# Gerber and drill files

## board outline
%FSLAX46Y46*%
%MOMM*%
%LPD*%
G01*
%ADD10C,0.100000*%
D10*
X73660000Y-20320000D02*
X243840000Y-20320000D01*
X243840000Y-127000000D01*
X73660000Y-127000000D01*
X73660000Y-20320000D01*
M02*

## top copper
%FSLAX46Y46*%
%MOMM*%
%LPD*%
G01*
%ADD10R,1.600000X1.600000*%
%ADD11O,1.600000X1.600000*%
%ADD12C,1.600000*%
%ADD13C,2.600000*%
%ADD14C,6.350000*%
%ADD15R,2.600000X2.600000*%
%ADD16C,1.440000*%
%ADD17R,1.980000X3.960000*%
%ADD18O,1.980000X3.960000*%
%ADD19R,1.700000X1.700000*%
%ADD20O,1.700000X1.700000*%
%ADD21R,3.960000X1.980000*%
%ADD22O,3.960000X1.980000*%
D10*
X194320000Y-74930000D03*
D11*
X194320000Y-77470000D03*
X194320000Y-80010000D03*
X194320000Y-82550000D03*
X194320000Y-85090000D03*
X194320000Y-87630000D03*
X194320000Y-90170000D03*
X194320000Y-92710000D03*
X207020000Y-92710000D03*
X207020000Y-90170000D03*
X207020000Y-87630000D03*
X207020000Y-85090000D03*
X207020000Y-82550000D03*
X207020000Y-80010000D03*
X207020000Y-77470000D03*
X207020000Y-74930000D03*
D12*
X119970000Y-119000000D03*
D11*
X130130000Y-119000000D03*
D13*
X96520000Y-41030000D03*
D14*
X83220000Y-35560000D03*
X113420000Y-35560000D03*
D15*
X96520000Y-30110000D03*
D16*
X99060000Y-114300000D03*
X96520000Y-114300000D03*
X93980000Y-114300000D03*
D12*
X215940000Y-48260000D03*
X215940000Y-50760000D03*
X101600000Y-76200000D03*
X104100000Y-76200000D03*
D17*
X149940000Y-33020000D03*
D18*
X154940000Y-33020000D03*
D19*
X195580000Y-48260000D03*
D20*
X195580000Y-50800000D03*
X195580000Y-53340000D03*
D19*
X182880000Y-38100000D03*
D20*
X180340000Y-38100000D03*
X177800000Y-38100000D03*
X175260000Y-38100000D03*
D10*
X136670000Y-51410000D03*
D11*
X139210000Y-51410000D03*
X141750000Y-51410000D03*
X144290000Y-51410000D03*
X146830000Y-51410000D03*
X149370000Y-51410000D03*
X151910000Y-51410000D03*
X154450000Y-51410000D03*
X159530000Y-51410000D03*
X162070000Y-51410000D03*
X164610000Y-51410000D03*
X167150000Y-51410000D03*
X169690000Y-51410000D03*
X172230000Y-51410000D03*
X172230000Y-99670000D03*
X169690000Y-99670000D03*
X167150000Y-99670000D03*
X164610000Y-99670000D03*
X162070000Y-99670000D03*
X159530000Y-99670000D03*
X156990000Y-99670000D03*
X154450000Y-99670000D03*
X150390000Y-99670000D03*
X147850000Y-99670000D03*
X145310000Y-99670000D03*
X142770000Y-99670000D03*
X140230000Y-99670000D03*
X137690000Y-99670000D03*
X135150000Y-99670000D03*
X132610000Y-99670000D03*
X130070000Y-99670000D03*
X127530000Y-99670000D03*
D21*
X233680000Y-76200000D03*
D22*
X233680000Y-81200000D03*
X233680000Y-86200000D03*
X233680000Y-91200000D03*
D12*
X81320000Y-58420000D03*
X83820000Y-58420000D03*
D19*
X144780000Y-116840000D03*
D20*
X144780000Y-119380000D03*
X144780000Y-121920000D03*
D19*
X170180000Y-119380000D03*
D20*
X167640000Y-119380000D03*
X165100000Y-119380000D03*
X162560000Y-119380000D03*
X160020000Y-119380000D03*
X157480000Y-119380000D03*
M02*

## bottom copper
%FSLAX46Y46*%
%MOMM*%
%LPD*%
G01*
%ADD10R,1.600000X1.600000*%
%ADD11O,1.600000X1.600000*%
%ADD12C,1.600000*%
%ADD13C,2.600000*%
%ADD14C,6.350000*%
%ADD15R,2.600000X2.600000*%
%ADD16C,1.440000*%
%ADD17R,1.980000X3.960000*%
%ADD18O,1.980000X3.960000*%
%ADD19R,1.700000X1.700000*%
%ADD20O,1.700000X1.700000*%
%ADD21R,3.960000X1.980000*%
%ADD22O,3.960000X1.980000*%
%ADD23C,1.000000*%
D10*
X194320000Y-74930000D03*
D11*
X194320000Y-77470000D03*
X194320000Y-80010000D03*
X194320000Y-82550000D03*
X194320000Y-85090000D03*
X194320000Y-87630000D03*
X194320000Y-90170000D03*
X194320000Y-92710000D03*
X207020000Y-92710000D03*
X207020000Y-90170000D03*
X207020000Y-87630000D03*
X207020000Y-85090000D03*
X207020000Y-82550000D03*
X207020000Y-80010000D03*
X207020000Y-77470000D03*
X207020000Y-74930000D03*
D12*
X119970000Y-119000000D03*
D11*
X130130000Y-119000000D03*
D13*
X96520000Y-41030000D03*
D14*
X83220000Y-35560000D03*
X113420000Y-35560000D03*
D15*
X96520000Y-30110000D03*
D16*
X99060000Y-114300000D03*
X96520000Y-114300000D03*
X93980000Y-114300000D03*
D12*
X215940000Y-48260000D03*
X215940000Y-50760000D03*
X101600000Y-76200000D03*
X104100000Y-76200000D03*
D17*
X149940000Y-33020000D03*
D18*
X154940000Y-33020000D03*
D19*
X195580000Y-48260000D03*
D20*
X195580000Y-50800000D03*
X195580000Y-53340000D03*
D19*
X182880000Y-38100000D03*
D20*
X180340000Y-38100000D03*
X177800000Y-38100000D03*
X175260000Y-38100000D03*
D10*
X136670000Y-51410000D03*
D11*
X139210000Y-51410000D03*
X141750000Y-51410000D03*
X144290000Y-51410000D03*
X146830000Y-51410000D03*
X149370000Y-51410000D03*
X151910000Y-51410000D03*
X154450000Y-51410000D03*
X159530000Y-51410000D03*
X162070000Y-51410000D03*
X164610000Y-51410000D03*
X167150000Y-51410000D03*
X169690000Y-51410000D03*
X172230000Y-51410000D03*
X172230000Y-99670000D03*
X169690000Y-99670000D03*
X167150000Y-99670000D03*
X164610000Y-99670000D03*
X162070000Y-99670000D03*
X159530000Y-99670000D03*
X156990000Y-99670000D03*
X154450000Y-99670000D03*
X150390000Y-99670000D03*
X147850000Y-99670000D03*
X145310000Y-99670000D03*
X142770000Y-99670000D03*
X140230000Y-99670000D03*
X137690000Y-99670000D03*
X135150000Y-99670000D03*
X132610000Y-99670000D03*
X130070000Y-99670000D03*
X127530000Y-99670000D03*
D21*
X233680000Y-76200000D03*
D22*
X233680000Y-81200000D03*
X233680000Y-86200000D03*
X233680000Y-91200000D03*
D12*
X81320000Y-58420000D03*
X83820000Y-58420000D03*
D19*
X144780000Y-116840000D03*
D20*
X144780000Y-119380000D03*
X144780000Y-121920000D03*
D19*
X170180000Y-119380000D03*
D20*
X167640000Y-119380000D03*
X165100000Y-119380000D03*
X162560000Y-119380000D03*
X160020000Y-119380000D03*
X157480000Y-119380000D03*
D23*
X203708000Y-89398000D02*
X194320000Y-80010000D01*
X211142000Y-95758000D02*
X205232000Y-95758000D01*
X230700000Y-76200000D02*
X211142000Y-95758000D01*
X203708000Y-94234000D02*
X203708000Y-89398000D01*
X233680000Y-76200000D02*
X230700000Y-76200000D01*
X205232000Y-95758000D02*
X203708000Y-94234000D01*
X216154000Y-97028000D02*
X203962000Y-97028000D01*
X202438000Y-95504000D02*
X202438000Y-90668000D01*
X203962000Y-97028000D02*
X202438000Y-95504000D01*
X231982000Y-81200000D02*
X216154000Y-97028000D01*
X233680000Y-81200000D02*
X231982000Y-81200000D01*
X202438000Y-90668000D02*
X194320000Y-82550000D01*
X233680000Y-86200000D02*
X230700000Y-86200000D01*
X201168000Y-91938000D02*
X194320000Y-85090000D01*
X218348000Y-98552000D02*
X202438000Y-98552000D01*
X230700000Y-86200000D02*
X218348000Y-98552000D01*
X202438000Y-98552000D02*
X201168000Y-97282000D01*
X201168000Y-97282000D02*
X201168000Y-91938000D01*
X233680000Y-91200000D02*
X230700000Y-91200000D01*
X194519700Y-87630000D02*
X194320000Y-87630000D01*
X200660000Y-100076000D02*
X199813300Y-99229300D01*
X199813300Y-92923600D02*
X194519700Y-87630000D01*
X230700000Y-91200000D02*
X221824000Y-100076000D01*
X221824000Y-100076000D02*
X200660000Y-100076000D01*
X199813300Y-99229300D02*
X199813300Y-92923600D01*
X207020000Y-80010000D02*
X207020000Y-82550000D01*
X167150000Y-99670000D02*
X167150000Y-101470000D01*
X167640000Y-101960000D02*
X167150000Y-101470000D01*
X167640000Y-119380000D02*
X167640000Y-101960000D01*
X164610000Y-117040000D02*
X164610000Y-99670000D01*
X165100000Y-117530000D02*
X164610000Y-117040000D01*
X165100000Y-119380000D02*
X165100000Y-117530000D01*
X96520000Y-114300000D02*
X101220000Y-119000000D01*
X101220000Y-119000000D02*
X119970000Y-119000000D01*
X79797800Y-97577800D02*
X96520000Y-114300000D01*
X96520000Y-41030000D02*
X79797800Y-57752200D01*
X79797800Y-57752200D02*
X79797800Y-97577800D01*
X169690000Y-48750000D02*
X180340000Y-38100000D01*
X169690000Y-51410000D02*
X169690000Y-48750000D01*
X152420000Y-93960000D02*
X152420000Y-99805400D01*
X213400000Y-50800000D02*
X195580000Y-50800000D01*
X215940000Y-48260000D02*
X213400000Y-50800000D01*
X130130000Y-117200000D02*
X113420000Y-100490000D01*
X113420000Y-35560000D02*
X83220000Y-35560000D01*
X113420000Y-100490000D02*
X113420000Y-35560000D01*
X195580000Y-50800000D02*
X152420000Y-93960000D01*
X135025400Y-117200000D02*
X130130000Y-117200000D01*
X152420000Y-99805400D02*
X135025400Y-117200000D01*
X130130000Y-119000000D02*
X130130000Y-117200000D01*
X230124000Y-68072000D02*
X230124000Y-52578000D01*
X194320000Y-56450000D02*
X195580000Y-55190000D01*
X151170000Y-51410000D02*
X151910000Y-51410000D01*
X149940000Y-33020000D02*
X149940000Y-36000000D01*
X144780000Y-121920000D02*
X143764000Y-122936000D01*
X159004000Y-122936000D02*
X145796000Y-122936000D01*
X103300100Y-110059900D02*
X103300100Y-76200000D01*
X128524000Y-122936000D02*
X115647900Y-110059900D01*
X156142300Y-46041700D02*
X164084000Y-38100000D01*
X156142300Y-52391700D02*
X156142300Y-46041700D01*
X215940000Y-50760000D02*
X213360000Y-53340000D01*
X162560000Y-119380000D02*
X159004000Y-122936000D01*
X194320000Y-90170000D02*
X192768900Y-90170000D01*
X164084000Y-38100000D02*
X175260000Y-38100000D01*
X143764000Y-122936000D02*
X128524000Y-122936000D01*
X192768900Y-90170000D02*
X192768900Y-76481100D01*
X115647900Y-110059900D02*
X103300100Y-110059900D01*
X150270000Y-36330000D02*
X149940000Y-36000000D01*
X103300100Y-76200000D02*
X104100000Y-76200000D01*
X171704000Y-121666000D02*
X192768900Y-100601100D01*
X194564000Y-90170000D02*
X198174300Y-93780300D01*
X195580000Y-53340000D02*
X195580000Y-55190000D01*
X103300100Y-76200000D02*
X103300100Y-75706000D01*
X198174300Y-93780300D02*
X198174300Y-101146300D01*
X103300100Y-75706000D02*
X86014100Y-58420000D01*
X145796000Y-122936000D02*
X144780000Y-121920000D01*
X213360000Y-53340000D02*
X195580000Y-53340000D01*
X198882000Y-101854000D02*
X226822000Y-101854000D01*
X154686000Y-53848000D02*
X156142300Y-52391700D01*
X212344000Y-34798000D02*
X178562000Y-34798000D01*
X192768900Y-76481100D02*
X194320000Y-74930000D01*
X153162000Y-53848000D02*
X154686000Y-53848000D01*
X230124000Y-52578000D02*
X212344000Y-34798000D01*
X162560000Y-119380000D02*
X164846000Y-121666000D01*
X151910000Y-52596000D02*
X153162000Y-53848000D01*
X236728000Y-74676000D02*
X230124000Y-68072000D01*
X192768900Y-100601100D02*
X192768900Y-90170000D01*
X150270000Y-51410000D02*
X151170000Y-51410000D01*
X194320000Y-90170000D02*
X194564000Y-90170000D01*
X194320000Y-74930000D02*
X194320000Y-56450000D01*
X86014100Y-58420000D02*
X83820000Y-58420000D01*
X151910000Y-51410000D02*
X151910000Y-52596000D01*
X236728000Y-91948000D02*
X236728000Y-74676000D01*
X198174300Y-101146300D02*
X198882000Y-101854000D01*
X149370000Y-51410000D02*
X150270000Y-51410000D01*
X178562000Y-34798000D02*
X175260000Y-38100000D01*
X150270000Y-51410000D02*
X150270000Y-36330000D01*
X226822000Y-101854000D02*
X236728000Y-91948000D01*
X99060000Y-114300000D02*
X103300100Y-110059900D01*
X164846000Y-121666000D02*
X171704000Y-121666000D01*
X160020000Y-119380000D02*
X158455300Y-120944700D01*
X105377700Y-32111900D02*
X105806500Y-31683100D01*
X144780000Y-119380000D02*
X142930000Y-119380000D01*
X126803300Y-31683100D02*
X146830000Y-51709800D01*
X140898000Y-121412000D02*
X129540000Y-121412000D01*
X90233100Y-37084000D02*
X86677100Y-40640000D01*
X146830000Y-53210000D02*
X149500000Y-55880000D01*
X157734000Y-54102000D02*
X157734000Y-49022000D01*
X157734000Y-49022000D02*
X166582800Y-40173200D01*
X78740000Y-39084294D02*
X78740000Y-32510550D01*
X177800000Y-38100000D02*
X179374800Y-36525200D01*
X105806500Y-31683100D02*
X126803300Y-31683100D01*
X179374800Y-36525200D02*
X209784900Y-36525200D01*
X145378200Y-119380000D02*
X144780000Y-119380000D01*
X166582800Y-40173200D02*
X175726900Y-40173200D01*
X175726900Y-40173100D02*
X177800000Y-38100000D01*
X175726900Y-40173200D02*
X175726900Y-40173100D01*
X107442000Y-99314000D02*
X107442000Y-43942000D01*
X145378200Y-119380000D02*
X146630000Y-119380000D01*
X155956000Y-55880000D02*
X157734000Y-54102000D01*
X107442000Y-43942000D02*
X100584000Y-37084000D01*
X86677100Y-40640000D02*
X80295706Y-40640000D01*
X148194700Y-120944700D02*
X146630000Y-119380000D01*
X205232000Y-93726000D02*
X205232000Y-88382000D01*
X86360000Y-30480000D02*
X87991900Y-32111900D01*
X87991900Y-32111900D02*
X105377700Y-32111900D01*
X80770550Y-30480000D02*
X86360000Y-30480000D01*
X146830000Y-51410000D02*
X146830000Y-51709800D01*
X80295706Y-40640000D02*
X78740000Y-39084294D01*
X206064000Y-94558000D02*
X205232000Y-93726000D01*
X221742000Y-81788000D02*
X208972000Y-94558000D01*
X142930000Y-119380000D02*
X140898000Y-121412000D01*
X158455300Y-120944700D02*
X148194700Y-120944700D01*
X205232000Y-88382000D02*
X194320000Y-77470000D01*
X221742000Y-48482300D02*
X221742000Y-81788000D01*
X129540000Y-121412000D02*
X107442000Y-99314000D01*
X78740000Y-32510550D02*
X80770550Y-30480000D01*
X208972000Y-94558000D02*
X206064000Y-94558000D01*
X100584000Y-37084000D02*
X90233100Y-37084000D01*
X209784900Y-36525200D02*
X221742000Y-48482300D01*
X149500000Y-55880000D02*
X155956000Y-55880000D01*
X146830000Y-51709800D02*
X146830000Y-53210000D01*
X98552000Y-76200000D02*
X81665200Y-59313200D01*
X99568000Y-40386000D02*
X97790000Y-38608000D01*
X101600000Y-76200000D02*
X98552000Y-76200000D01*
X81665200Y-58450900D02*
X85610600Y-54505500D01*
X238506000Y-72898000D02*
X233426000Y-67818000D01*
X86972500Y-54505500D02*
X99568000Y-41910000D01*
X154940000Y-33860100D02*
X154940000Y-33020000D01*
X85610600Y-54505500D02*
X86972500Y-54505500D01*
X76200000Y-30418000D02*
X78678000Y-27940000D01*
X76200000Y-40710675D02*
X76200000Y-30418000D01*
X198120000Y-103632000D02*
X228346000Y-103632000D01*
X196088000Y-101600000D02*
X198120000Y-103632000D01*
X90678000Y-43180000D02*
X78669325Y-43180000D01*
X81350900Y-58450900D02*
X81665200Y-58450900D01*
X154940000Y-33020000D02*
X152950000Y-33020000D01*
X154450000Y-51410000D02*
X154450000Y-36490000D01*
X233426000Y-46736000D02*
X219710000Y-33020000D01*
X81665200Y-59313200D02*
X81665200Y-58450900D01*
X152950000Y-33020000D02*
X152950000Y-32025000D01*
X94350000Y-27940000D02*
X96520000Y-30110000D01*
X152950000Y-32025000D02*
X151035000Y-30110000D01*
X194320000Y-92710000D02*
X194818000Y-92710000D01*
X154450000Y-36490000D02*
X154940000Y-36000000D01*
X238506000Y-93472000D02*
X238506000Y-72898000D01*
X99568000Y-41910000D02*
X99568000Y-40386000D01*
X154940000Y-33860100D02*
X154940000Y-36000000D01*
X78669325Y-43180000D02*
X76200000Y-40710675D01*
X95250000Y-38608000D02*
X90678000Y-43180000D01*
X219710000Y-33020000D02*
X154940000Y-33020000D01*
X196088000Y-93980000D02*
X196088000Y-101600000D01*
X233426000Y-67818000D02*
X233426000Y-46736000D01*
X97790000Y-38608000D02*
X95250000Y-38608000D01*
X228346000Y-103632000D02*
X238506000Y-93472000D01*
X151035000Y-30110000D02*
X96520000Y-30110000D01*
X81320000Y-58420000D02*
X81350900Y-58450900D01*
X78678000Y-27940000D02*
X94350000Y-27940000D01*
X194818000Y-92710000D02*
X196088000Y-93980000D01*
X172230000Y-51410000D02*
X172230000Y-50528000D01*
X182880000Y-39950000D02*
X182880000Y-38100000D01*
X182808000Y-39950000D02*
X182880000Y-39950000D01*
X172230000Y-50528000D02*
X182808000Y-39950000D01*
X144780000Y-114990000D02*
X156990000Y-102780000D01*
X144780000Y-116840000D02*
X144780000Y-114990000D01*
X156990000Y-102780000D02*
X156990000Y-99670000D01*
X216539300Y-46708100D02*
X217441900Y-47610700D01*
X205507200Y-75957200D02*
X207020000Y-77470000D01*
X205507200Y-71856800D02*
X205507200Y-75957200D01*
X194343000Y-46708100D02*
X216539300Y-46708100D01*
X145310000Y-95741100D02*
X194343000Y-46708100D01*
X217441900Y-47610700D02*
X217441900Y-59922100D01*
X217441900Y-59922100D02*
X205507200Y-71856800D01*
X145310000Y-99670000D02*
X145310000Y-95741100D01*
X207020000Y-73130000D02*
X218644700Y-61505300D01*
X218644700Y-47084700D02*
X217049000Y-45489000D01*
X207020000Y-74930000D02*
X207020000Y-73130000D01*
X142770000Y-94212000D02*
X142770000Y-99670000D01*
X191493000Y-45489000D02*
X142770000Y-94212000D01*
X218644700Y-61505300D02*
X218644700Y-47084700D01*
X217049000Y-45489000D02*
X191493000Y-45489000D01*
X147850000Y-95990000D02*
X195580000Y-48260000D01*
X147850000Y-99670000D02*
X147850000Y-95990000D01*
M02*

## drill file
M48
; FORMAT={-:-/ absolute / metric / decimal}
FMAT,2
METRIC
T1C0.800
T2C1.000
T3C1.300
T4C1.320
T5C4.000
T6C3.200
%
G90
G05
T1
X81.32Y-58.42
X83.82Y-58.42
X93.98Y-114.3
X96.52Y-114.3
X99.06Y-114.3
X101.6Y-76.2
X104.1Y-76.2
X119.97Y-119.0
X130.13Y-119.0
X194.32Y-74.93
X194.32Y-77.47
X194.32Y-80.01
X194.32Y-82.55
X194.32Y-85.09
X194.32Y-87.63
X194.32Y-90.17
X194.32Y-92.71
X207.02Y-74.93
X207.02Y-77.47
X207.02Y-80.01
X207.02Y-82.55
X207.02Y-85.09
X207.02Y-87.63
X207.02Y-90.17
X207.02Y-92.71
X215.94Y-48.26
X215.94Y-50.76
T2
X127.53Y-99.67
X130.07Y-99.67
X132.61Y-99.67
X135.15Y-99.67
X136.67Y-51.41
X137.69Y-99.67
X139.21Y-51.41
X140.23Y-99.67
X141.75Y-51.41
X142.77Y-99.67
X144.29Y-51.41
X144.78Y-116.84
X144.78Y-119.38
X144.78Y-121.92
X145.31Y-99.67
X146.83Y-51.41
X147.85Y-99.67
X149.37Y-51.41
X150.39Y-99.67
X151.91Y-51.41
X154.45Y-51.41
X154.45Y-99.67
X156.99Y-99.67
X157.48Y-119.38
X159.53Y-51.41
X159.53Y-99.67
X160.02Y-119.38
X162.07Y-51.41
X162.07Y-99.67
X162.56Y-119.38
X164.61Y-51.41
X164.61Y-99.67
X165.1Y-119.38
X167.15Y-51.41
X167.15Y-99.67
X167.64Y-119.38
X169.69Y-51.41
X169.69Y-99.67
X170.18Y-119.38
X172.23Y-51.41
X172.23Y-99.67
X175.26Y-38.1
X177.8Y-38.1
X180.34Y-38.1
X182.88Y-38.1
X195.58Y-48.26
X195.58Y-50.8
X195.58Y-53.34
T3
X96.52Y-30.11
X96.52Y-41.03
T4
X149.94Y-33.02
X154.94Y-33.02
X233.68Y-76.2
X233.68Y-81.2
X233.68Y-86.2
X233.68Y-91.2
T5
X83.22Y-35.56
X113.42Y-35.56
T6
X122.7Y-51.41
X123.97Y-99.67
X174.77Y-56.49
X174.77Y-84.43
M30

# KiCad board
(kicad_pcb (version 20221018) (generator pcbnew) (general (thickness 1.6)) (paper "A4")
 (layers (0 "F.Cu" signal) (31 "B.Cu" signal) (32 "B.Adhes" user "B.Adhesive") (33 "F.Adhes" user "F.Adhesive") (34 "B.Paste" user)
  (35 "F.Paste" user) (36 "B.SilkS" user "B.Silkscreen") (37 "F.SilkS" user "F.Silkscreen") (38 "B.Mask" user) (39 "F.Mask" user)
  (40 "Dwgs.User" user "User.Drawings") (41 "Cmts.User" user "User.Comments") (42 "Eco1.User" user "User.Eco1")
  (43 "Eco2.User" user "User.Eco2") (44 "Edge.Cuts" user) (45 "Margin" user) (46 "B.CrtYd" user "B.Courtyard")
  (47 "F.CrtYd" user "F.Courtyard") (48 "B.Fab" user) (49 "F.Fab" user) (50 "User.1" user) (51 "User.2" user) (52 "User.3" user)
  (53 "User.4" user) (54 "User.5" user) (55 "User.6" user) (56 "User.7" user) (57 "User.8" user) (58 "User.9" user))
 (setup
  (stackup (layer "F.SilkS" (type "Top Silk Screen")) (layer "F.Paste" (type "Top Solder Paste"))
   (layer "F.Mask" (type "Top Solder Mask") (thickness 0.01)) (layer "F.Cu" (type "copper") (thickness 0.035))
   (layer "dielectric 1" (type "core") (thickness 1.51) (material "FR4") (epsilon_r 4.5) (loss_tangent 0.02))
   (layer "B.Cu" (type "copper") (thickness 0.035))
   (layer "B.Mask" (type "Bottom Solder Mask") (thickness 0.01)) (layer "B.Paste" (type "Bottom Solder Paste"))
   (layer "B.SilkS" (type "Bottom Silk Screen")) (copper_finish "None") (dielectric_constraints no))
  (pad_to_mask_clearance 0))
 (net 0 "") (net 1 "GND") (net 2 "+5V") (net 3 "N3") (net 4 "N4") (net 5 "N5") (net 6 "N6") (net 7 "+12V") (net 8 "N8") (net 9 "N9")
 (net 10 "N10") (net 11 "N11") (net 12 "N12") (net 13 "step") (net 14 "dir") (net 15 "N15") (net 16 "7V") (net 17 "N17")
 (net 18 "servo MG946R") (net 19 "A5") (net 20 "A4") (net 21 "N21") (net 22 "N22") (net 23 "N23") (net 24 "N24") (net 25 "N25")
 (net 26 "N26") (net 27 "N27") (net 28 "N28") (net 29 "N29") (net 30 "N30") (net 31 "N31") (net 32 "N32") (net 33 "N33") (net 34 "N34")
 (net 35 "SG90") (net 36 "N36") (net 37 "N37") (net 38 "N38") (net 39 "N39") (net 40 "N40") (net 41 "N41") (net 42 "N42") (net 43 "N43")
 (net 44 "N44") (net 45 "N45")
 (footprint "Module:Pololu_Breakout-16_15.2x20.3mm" (layer "F.Cu") (at 194.32 74.93)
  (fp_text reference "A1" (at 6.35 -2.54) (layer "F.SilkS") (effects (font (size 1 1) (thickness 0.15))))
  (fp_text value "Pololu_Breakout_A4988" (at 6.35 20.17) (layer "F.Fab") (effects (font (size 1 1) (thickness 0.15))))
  (pad "1" thru_hole rect (at 0 0) (size 1.6 1.6) (drill 0.8) (layers "*.Cu" "*.Mask") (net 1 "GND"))
  (pad "2" thru_hole oval (at 0 2.54) (size 1.6 1.6) (drill 0.8) (layers "*.Cu" "*.Mask") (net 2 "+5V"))
  (pad "3" thru_hole oval (at 0 5.08) (size 1.6 1.6) (drill 0.8) (layers "*.Cu" "*.Mask") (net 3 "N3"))
  (pad "4" thru_hole oval (at 0 7.62) (size 1.6 1.6) (drill 0.8) (layers "*.Cu" "*.Mask") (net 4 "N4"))
  (pad "5" thru_hole oval (at 0 10.16) (size 1.6 1.6) (drill 0.8) (layers "*.Cu" "*.Mask") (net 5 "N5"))
  (pad "6" thru_hole oval (at 0 12.7) (size 1.6 1.6) (drill 0.8) (layers "*.Cu" "*.Mask") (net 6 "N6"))
  (pad "7" thru_hole oval (at 0 15.24) (size 1.6 1.6) (drill 0.8) (layers "*.Cu" "*.Mask") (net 1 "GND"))
  (pad "8" thru_hole oval (at 0 17.78) (size 1.6 1.6) (drill 0.8) (layers "*.Cu" "*.Mask") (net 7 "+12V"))
  (pad "9" thru_hole oval (at 12.7 17.78) (size 1.6 1.6) (drill 0.8) (layers "*.Cu" "*.Mask") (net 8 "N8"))
  (pad "10" thru_hole oval (at 12.7 15.24) (size 1.6 1.6) (drill 0.8) (layers "*.Cu" "*.Mask") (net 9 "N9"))
  (pad "11" thru_hole oval (at 12.7 12.7) (size 1.6 1.6) (drill 0.8) (layers "*.Cu" "*.Mask") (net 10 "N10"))
  (pad "12" thru_hole oval (at 12.7 10.16) (size 1.6 1.6) (drill 0.8) (layers "*.Cu" "*.Mask") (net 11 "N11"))
  (pad "13" thru_hole oval (at 12.7 7.62) (size 1.6 1.6) (drill 0.8) (layers "*.Cu" "*.Mask") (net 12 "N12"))
  (pad "14" thru_hole oval (at 12.7 5.08) (size 1.6 1.6) (drill 0.8) (layers "*.Cu" "*.Mask") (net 12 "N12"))
  (pad "15" thru_hole oval (at 12.7 2.54) (size 1.6 1.6) (drill 0.8) (layers "*.Cu" "*.Mask") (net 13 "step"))
  (pad "16" thru_hole oval (at 12.7 0) (size 1.6 1.6) (drill 0.8) (layers "*.Cu" "*.Mask") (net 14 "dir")))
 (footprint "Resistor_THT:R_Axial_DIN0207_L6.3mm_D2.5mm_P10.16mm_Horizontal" (layer "F.Cu") (at 119.97 119)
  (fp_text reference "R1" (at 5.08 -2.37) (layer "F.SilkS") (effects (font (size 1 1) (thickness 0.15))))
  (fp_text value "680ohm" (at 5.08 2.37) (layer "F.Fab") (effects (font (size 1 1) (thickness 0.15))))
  (pad "1" thru_hole circle (at 0 0) (size 1.6 1.6) (drill 0.8) (layers "*.Cu" "*.Mask") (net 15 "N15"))
  (pad "2" thru_hole oval (at 10.16 0) (size 1.6 1.6) (drill 0.8) (layers "*.Cu" "*.Mask") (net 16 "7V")))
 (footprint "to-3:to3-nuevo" (layer "F.Cu") (at 98.74 32.39)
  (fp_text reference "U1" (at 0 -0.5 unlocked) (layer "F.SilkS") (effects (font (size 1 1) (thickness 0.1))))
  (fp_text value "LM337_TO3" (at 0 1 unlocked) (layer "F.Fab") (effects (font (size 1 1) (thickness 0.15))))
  (pad "1" thru_hole circle (at -2.22 8.64) (size 2.6 2.6) (drill 1.3) (layers "*.Cu" "*.Mask") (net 15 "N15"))
  (pad "2" thru_hole circle (at -15.52 3.17) (size 6.35 6.35) (drill 4) (layers "*.Cu" "*.Mask") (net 16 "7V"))
  (pad "2" thru_hole circle (at 14.68 3.17) (size 6.35 6.35) (drill 4) (layers "*.Cu" "*.Mask") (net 16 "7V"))
  (pad "3" thru_hole rect (at -2.22 -2.28) (size 2.6 2.6) (drill 1.3) (layers "*.Cu" "*.Mask") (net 7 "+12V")))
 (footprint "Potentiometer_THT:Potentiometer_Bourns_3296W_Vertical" (layer "F.Cu") (at 99.06 114.3)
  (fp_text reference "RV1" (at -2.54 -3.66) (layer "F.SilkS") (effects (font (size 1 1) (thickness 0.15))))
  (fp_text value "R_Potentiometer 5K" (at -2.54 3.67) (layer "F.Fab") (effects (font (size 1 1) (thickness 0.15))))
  (pad "1" thru_hole circle (at 0 0) (size 1.44 1.44) (drill 0.8) (layers "*.Cu" "*.Mask") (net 1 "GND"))
  (pad "2" thru_hole circle (at -2.54 0) (size 1.44 1.44) (drill 0.8) (layers "*.Cu" "*.Mask") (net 15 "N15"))
  (pad "3" thru_hole circle (at -5.08 0) (size 1.44 1.44) (drill 0.8) (layers "*.Cu" "*.Mask") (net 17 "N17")))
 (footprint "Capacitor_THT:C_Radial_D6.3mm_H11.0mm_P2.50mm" (layer "F.Cu") (at 215.94 48.26 -90)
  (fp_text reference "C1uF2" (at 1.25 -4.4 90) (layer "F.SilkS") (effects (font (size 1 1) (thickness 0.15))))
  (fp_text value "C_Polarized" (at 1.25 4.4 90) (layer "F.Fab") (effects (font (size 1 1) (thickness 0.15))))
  (pad "1" thru_hole circle (at 0 0 270) (size 1.6 1.6) (drill 0.8) (layers "*.Cu" "*.Mask") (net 16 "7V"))
  (pad "2" thru_hole circle (at 2.5 0 270) (size 1.6 1.6) (drill 0.8) (layers "*.Cu" "*.Mask") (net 1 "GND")))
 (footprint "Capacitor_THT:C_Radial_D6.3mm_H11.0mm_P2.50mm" (layer "F.Cu") (at 101.6 76.2)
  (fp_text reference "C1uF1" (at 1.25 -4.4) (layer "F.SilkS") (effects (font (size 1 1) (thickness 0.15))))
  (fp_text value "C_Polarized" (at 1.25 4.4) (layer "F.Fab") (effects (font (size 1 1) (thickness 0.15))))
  (pad "1" thru_hole circle (at 0 0) (size 1.6 1.6) (drill 0.8) (layers "*.Cu" "*.Mask") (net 7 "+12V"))
  (pad "2" thru_hole circle (at 2.5 0) (size 1.6 1.6) (drill 0.8) (layers "*.Cu" "*.Mask") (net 1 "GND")))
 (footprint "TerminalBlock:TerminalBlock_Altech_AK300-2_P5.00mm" (layer "F.Cu") (at 149.94 33.02)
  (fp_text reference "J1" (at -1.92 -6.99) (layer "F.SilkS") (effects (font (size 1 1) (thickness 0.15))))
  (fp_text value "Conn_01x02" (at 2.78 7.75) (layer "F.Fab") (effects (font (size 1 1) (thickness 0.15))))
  (pad "1" thru_hole rect (at 0 0) (size 1.98 3.96) (drill 1.32) (layers "*.Cu" "*.Mask") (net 1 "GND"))
  (pad "2" thru_hole oval (at 5 0) (size 1.98 3.96) (drill 1.32) (layers "*.Cu" "*.Mask") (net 7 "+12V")))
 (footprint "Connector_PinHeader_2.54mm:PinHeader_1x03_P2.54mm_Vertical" (layer "F.Cu") (at 195.58 48.26)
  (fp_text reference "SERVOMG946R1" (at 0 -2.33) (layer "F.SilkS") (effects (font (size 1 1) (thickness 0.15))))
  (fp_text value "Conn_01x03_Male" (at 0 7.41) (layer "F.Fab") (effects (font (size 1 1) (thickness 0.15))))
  (pad "1" thru_hole rect (at 0 0) (size 1.7 1.7) (drill 1) (layers "*.Cu" "*.Mask") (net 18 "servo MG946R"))
  (pad "2" thru_hole oval (at 0 2.54) (size 1.7 1.7) (drill 1) (layers "*.Cu" "*.Mask") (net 16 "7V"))
  (pad "3" thru_hole oval (at 0 5.08) (size 1.7 1.7) (drill 1) (layers "*.Cu" "*.Mask") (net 1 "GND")))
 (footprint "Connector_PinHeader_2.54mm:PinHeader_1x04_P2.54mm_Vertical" (layer "F.Cu") (at 182.88 38.1 -90)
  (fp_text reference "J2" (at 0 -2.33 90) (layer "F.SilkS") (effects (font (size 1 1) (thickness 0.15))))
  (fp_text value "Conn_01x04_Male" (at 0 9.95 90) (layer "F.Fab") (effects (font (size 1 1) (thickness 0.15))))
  (pad "1" thru_hole rect (at 0 0 270) (size 1.7 1.7) (drill 1) (layers "*.Cu" "*.Mask") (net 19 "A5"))
  (pad "2" thru_hole oval (at 0 2.54 270) (size 1.7 1.7) (drill 1) (layers "*.Cu" "*.Mask") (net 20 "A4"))
  (pad "3" thru_hole oval (at 0 5.08 270) (size 1.7 1.7) (drill 1) (layers "*.Cu" "*.Mask") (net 2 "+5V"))
  (pad "4" thru_hole oval (at 0 7.62 270) (size 1.7 1.7) (drill 1) (layers "*.Cu" "*.Mask") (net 1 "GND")))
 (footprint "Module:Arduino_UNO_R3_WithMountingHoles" (layer "F.Cu") (at 136.67 51.41)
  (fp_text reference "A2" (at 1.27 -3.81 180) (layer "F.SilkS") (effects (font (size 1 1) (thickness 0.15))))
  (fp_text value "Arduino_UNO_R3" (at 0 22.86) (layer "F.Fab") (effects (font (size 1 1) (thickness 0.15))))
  (pad "" np_thru_hole circle (at -13.97 0 90) (size 3.2 3.2) (drill 3.2) (layers "*.Cu" "*.Mask"))
  (pad "" np_thru_hole circle (at -12.7 48.26 90) (size 3.2 3.2) (drill 3.2) (layers "*.Cu" "*.Mask"))
  (pad "" np_thru_hole circle (at 38.1 5.08 90) (size 3.2 3.2) (drill 3.2) (layers "*.Cu" "*.Mask"))
  (pad "" np_thru_hole circle (at 38.1 33.02 90) (size 3.2 3.2) (drill 3.2) (layers "*.Cu" "*.Mask"))
  (pad "1" thru_hole rect (at 0 0 90) (size 1.6 1.6) (drill 1) (layers "*.Cu" "*.Mask") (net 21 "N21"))
  (pad "2" thru_hole oval (at 2.54 0 90) (size 1.6 1.6) (drill 1) (layers "*.Cu" "*.Mask") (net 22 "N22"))
  (pad "3" thru_hole oval (at 5.08 0 90) (size 1.6 1.6) (drill 1) (layers "*.Cu" "*.Mask") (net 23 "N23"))
  (pad "4" thru_hole oval (at 7.62 0 90) (size 1.6 1.6) (drill 1) (layers "*.Cu" "*.Mask") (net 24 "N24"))
  (pad "5" thru_hole oval (at 10.16 0 90) (size 1.6 1.6) (drill 1) (layers "*.Cu" "*.Mask") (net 2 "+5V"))
  (pad "6" thru_hole oval (at 12.7 0 90) (size 1.6 1.6) (drill 1) (layers "*.Cu" "*.Mask") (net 1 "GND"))
  (pad "7" thru_hole oval (at 15.24 0 90) (size 1.6 1.6) (drill 1) (layers "*.Cu" "*.Mask") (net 1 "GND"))
  (pad "8" thru_hole oval (at 17.78 0 90) (size 1.6 1.6) (drill 1) (layers "*.Cu" "*.Mask") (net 7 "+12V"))
  (pad "9" thru_hole oval (at 22.86 0 90) (size 1.6 1.6) (drill 1) (layers "*.Cu" "*.Mask") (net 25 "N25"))
  (pad "10" thru_hole oval (at 25.4 0 90) (size 1.6 1.6) (drill 1) (layers "*.Cu" "*.Mask") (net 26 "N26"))
  (pad "11" thru_hole oval (at 27.94 0 90) (size 1.6 1.6) (drill 1) (layers "*.Cu" "*.Mask") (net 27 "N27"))
  (pad "12" thru_hole oval (at 30.48 0 90) (size 1.6 1.6) (drill 1) (layers "*.Cu" "*.Mask") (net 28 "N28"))
  (pad "13" thru_hole oval (at 33.02 0 90) (size 1.6 1.6) (drill 1) (layers "*.Cu" "*.Mask") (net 20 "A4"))
  (pad "14" thru_hole oval (at 35.56 0 90) (size 1.6 1.6) (drill 1) (layers "*.Cu" "*.Mask") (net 19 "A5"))
  (pad "15" thru_hole oval (at 35.56 48.26 90) (size 1.6 1.6) (drill 1) (layers "*.Cu" "*.Mask") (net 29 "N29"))
  (pad "16" thru_hole oval (at 33.02 48.26 90) (size 1.6 1.6) (drill 1) (layers "*.Cu" "*.Mask") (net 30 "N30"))
  (pad "17" thru_hole oval (at 30.48 48.26 90) (size 1.6 1.6) (drill 1) (layers "*.Cu" "*.Mask") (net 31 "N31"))
  (pad "18" thru_hole oval (at 27.94 48.26 90) (size 1.6 1.6) (drill 1) (layers "*.Cu" "*.Mask") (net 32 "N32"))
  (pad "19" thru_hole oval (at 25.4 48.26 90) (size 1.6 1.6) (drill 1) (layers "*.Cu" "*.Mask") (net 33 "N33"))
  (pad "20" thru_hole oval (at 22.86 48.26 90) (size 1.6 1.6) (drill 1) (layers "*.Cu" "*.Mask") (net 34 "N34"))
  (pad "21" thru_hole oval (at 20.32 48.26 90) (size 1.6 1.6) (drill 1) (layers "*.Cu" "*.Mask") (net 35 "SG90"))
  (pad "22" thru_hole oval (at 17.78 48.26 90) (size 1.6 1.6) (drill 1) (layers "*.Cu" "*.Mask") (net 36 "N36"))
  (pad "23" thru_hole oval (at 13.72 48.26 90) (size 1.6 1.6) (drill 1) (layers "*.Cu" "*.Mask") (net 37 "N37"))
  (pad "24" thru_hole oval (at 11.18 48.26 90) (size 1.6 1.6) (drill 1) (layers "*.Cu" "*.Mask") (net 18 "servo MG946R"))
  (pad "25" thru_hole oval (at 8.64 48.26 90) (size 1.6 1.6) (drill 1) (layers "*.Cu" "*.Mask") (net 13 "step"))
  (pad "26" thru_hole oval (at 6.1 48.26 90) (size 1.6 1.6) (drill 1) (layers "*.Cu" "*.Mask") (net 14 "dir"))
  (pad "27" thru_hole oval (at 3.56 48.26 90) (size 1.6 1.6) (drill 1) (layers "*.Cu" "*.Mask") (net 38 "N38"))
  (pad "28" thru_hole oval (at 1.02 48.26 90) (size 1.6 1.6) (drill 1) (layers "*.Cu" "*.Mask") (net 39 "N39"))
  (pad "29" thru_hole oval (at -1.52 48.26 90) (size 1.6 1.6) (drill 1) (layers "*.Cu" "*.Mask") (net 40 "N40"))
  (pad "30" thru_hole oval (at -4.06 48.26 90) (size 1.6 1.6) (drill 1) (layers "*.Cu" "*.Mask") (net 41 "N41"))
  (pad "31" thru_hole oval (at -6.6 48.26 90) (size 1.6 1.6) (drill 1) (layers "*.Cu" "*.Mask") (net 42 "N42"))
  (pad "32" thru_hole oval (at -9.14 48.26 90) (size 1.6 1.6) (drill 1) (layers "*.Cu" "*.Mask") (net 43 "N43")))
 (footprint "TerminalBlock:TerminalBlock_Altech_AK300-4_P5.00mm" (layer "F.Cu") (at 233.68 76.2 -90)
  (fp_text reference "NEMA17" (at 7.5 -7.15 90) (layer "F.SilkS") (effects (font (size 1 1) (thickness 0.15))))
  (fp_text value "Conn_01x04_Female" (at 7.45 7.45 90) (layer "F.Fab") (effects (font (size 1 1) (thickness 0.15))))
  (pad "1" thru_hole rect (at 0 0 270) (size 1.98 3.96) (drill 1.32) (layers "*.Cu" "*.Mask") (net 3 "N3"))
  (pad "2" thru_hole oval (at 5 0 270) (size 1.98 3.96) (drill 1.32) (layers "*.Cu" "*.Mask") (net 4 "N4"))
  (pad "3" thru_hole oval (at 10 0 270) (size 1.98 3.96) (drill 1.32) (layers "*.Cu" "*.Mask") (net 5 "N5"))
  (pad "4" thru_hole oval (at 15 0 270) (size 1.98 3.96) (drill 1.32) (layers "*.Cu" "*.Mask") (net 6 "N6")))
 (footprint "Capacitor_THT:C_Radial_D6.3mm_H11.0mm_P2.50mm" (layer "F.Cu") (at 81.32 58.42)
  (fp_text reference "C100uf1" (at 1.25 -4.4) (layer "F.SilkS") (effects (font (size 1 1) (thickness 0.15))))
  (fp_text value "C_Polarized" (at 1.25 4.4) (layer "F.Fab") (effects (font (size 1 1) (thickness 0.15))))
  (pad "1" thru_hole circle (at 0 0) (size 1.6 1.6) (drill 0.8) (layers "*.Cu" "*.Mask") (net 7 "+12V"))
  (pad "2" thru_hole circle (at 2.5 0) (size 1.6 1.6) (drill 0.8) (layers "*.Cu" "*.Mask") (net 1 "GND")))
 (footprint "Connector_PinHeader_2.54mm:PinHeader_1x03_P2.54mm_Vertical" (layer "F.Cu") (at 144.78 116.84)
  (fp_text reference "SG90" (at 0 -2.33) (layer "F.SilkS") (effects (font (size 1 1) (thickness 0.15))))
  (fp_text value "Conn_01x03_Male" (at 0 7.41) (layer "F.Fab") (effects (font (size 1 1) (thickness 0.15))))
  (pad "1" thru_hole rect (at 0 0) (size 1.7 1.7) (drill 1) (layers "*.Cu" "*.Mask") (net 35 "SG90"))
  (pad "2" thru_hole oval (at 0 2.54) (size 1.7 1.7) (drill 1) (layers "*.Cu" "*.Mask") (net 2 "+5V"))
  (pad "3" thru_hole oval (at 0 5.08) (size 1.7 1.7) (drill 1) (layers "*.Cu" "*.Mask") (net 1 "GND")))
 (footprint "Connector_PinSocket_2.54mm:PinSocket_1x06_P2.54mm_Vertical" (layer "F.Cu") (at 170.18 119.38 -90)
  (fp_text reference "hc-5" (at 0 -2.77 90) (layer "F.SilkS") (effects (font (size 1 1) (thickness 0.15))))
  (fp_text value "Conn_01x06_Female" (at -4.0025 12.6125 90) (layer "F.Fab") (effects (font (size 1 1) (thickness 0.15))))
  (pad "1" thru_hole rect (at 0 0 270) (size 1.7 1.7) (drill 1) (layers "*.Cu" "*.Mask") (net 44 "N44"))
  (pad "2" thru_hole oval (at 0 2.54 270) (size 1.7 1.7) (drill 1) (layers "*.Cu" "*.Mask") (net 31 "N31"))
  (pad "3" thru_hole oval (at 0 5.08 270) (size 1.7 1.7) (drill 1) (layers "*.Cu" "*.Mask") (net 32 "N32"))
  (pad "4" thru_hole oval (at 0 7.62 270) (size 1.7 1.7) (drill 1) (layers "*.Cu" "*.Mask") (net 1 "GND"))
  (pad "5" thru_hole oval (at 0 10.16 270) (size 1.7 1.7) (drill 1) (layers "*.Cu" "*.Mask") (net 2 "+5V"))
  (pad "6" thru_hole oval (at 0 12.7 270) (size 1.7 1.7) (drill 1) (layers "*.Cu" "*.Mask") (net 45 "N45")))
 (gr_rect (start 73.66 20.32) (end 243.84 127) (stroke (width 0.1) (type default)) (fill none) (layer "Edge.Cuts"))
 (segment (start 203.708 89.398) (end 194.32 80.01) (width 1) (layer "B.Cu") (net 3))
 (segment (start 211.142 95.758) (end 205.232 95.758) (width 1) (layer "B.Cu") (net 3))
 (segment (start 230.7 76.2) (end 211.142 95.758) (width 1) (layer "B.Cu") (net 3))
 (segment (start 203.708 94.234) (end 203.708 89.398) (width 1) (layer "B.Cu") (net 3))
 (segment (start 233.68 76.2) (end 230.7 76.2) (width 1) (layer "B.Cu") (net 3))
 (segment (start 205.232 95.758) (end 203.708 94.234) (width 1) (layer "B.Cu") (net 3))
 (segment (start 216.154 97.028) (end 203.962 97.028) (width 1) (layer "B.Cu") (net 4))
 (segment (start 202.438 95.504) (end 202.438 90.668) (width 1) (layer "B.Cu") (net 4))
 (segment (start 203.962 97.028) (end 202.438 95.504) (width 1) (layer "B.Cu") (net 4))
 (segment (start 231.982 81.2) (end 216.154 97.028) (width 1) (layer "B.Cu") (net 4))
 (segment (start 233.68 81.2) (end 231.982 81.2) (width 1) (layer "B.Cu") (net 4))
 (segment (start 202.438 90.668) (end 194.32 82.55) (width 1) (layer "B.Cu") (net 4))
 (segment (start 233.68 86.2) (end 230.7 86.2) (width 1) (layer "B.Cu") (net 5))
 (segment (start 201.168 91.938) (end 194.32 85.09) (width 1) (layer "B.Cu") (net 5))
 (segment (start 218.348 98.552) (end 202.438 98.552) (width 1) (layer "B.Cu") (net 5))
 (segment (start 230.7 86.2) (end 218.348 98.552) (width 1) (layer "B.Cu") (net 5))
 (segment (start 202.438 98.552) (end 201.168 97.282) (width 1) (layer "B.Cu") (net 5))
 (segment (start 201.168 97.282) (end 201.168 91.938) (width 1) (layer "B.Cu") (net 5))
 (segment (start 233.68 91.2) (end 230.7 91.2) (width 1) (layer "B.Cu") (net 6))
 (segment (start 194.5197 87.63) (end 194.32 87.63) (width 1) (layer "B.Cu") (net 6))
 (segment (start 200.66 100.076) (end 199.8133 99.2293) (width 1) (layer "B.Cu") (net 6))
 (segment (start 199.8133 92.9236) (end 194.5197 87.63) (width 1) (layer "B.Cu") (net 6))
 (segment (start 230.7 91.2) (end 221.824 100.076) (width 1) (layer "B.Cu") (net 6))
 (segment (start 221.824 100.076) (end 200.66 100.076) (width 1) (layer "B.Cu") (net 6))
 (segment (start 199.8133 99.2293) (end 199.8133 92.9236) (width 1) (layer "B.Cu") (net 6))
 (segment (start 207.02 80.01) (end 207.02 82.55) (width 1) (layer "B.Cu") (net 12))
 (segment (start 167.15 99.67) (end 167.15 101.47) (width 1) (layer "B.Cu") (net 31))
 (segment (start 167.64 101.96) (end 167.15 101.47) (width 1) (layer "B.Cu") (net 31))
 (segment (start 167.64 119.38) (end 167.64 101.96) (width 1) (layer "B.Cu") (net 31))
 (segment (start 164.61 117.04) (end 164.61 99.67) (width 1) (layer "B.Cu") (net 32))
 (segment (start 165.1 117.53) (end 164.61 117.04) (width 1) (layer "B.Cu") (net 32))
 (segment (start 165.1 119.38) (end 165.1 117.53) (width 1) (layer "B.Cu") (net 32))
 (segment (start 96.52 114.3) (end 101.22 119) (width 1) (layer "B.Cu") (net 15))
 (segment (start 101.22 119) (end 119.97 119) (width 1) (layer "B.Cu") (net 15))
 (segment (start 79.7978 97.5778) (end 96.52 114.3) (width 1) (layer "B.Cu") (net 15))
 (segment (start 96.52 41.03) (end 79.7978 57.7522) (width 1) (layer "B.Cu") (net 15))
 (segment (start 79.7978 57.7522) (end 79.7978 97.5778) (width 1) (layer "B.Cu") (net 15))
 (segment (start 169.69 48.75) (end 180.34 38.1) (width 1) (layer "B.Cu") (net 20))
 (segment (start 169.69 51.41) (end 169.69 48.75) (width 1) (layer "B.Cu") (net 20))
 (segment (start 152.42 93.96) (end 152.42 99.8054) (width 1) (layer "B.Cu") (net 16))
 (segment (start 213.4 50.8) (end 195.58 50.8) (width 1) (layer "B.Cu") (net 16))
 (segment (start 215.94 48.26) (end 213.4 50.8) (width 1) (layer "B.Cu") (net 16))
 (segment (start 130.13 117.2) (end 113.42 100.49) (width 1) (layer "B.Cu") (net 16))
 (segment (start 113.42 35.56) (end 83.22 35.56) (width 1) (layer "B.Cu") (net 16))
 (segment (start 113.42 100.49) (end 113.42 35.56) (width 1) (layer "B.Cu") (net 16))
 (segment (start 195.58 50.8) (end 152.42 93.96) (width 1) (layer "B.Cu") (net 16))
 (segment (start 135.0254 117.2) (end 130.13 117.2) (width 1) (layer "B.Cu") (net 16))
 (segment (start 152.42 99.8054) (end 135.0254 117.2) (width 1) (layer "B.Cu") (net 16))
 (segment (start 130.13 119) (end 130.13 117.2) (width 1) (layer "B.Cu") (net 16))
 (segment (start 230.124 68.072) (end 230.124 52.578) (width 1) (layer "B.Cu") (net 1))
 (segment (start 194.32 56.45) (end 195.58 55.19) (width 1) (layer "B.Cu") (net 1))
 (segment (start 151.17 51.41) (end 151.91 51.41) (width 1) (layer "B.Cu") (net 1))
 (segment (start 149.94 33.02) (end 149.94 36) (width 1) (layer "B.Cu") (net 1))
 (segment (start 144.78 121.92) (end 143.764 122.936) (width 1) (layer "B.Cu") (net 1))
 (segment (start 159.004 122.936) (end 145.796 122.936) (width 1) (layer "B.Cu") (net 1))
 (segment (start 103.3001 110.0599) (end 103.3001 76.2) (width 1) (layer "B.Cu") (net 1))
 (segment (start 128.524 122.936) (end 115.6479 110.0599) (width 1) (layer "B.Cu") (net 1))
 (segment (start 156.1423 46.0417) (end 164.084 38.1) (width 1) (layer "B.Cu") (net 1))
 (segment (start 156.1423 52.3917) (end 156.1423 46.0417) (width 1) (layer "B.Cu") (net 1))
 (segment (start 215.94 50.76) (end 213.36 53.34) (width 1) (layer "B.Cu") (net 1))
 (segment (start 162.56 119.38) (end 159.004 122.936) (width 1) (layer "B.Cu") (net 1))
 (segment (start 194.32 90.17) (end 192.7689 90.17) (width 1) (layer "B.Cu") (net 1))
 (segment (start 164.084 38.1) (end 175.26 38.1) (width 1) (layer "B.Cu") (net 1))
 (segment (start 143.764 122.936) (end 128.524 122.936) (width 1) (layer "B.Cu") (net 1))
 (segment (start 192.7689 90.17) (end 192.7689 76.4811) (width 1) (layer "B.Cu") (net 1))
 (segment (start 115.6479 110.0599) (end 103.3001 110.0599) (width 1) (layer "B.Cu") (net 1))
 (segment (start 150.27 36.33) (end 149.94 36) (width 1) (layer "B.Cu") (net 1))
 (segment (start 103.3001 76.2) (end 104.1 76.2) (width 1) (layer "B.Cu") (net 1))
 (segment (start 171.704 121.666) (end 192.7689 100.6011) (width 1) (layer "B.Cu") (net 1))
 (segment (start 194.564 90.17) (end 198.1743 93.7803) (width 1) (layer "B.Cu") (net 1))
 (segment (start 195.58 53.34) (end 195.58 55.19) (width 1) (layer "B.Cu") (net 1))
 (segment (start 103.3001 76.2) (end 103.3001 75.706) (width 1) (layer "B.Cu") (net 1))
 (segment (start 198.1743 93.7803) (end 198.1743 101.1463) (width 1) (layer "B.Cu") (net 1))
 (segment (start 103.3001 75.706) (end 86.0141 58.42) (width 1) (layer "B.Cu") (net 1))
 (segment (start 145.796 122.936) (end 144.78 121.92) (width 1) (layer "B.Cu") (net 1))
 (segment (start 213.36 53.34) (end 195.58 53.34) (width 1) (layer "B.Cu") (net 1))
 (segment (start 198.882 101.854) (end 226.822 101.854) (width 1) (layer "B.Cu") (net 1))
 (segment (start 154.686 53.848) (end 156.1423 52.3917) (width 1) (layer "B.Cu") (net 1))
 (segment (start 212.344 34.798) (end 178.562 34.798) (width 1) (layer "B.Cu") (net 1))
 (segment (start 192.7689 76.4811) (end 194.32 74.93) (width 1) (layer "B.Cu") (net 1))
 (segment (start 153.162 53.848) (end 154.686 53.848) (width 1) (layer "B.Cu") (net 1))
 (segment (start 230.124 52.578) (end 212.344 34.798) (width 1) (layer "B.Cu") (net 1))
 (segment (start 162.56 119.38) (end 164.846 121.666) (width 1) (layer "B.Cu") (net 1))
 (segment (start 151.91 52.596) (end 153.162 53.848) (width 1) (layer "B.Cu") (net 1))
 (segment (start 236.728 74.676) (end 230.124 68.072) (width 1) (layer "B.Cu") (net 1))
 (segment (start 192.7689 100.6011) (end 192.7689 90.17) (width 1) (layer "B.Cu") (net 1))
 (segment (start 150.27 51.41) (end 151.17 51.41) (width 1) (layer "B.Cu") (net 1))
 (segment (start 194.32 90.17) (end 194.564 90.17) (width 1) (layer "B.Cu") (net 1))
 (segment (start 194.32 74.93) (end 194.32 56.45) (width 1) (layer "B.Cu") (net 1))
 (segment (start 86.0141 58.42) (end 83.82 58.42) (width 1) (layer "B.Cu") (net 1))
 (segment (start 151.91 51.41) (end 151.91 52.596) (width 1) (layer "B.Cu") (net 1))
 (segment (start 236.728 91.948) (end 236.728 74.676) (width 1) (layer "B.Cu") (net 1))
 (segment (start 198.1743 101.1463) (end 198.882 101.854) (width 1) (layer "B.Cu") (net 1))
 (segment (start 149.37 51.41) (end 150.27 51.41) (width 1) (layer "B.Cu") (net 1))
 (segment (start 178.562 34.798) (end 175.26 38.1) (width 1) (layer "B.Cu") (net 1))
 (segment (start 150.27 51.41) (end 150.27 36.33) (width 1) (layer "B.Cu") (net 1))
 (segment (start 226.822 101.854) (end 236.728 91.948) (width 1) (layer "B.Cu") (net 1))
 (segment (start 99.06 114.3) (end 103.3001 110.0599) (width 1) (layer "B.Cu") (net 1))
 (segment (start 164.846 121.666) (end 171.704 121.666) (width 1) (layer "B.Cu") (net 1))
 (segment (start 160.02 119.38) (end 158.4553 120.9447) (width 1) (layer "B.Cu") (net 2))
 (segment (start 105.3777 32.1119) (end 105.8065 31.6831) (width 1) (layer "B.Cu") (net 2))
 (segment (start 144.78 119.38) (end 142.93 119.38) (width 1) (layer "B.Cu") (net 2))
 (segment (start 126.8033 31.6831) (end 146.83 51.7098) (width 1) (layer "B.Cu") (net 2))
 (segment (start 140.898 121.412) (end 129.54 121.412) (width 1) (layer "B.Cu") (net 2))
 (segment (start 90.2331 37.084) (end 86.6771 40.64) (width 1) (layer "B.Cu") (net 2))
 (segment (start 146.83 53.21) (end 149.5 55.88) (width 1) (layer "B.Cu") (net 2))
 (segment (start 157.734 54.102) (end 157.734 49.022) (width 1) (layer "B.Cu") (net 2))
 (segment (start 157.734 49.022) (end 166.5828 40.1732) (width 1) (layer "B.Cu") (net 2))
 (segment (start 78.74 39.084294) (end 78.74 32.51055) (width 1) (layer "B.Cu") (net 2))
 (segment (start 177.8 38.1) (end 179.3748 36.5252) (width 1) (layer "B.Cu") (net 2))
 (segment (start 105.8065 31.6831) (end 126.8033 31.6831) (width 1) (layer "B.Cu") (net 2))
 (segment (start 179.3748 36.5252) (end 209.7849 36.5252) (width 1) (layer "B.Cu") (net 2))
 (segment (start 145.3782 119.38) (end 144.78 119.38) (width 1) (layer "B.Cu") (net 2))
 (segment (start 166.5828 40.1732) (end 175.7269 40.1732) (width 1) (layer "B.Cu") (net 2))
 (segment (start 175.7269 40.1731) (end 177.8 38.1) (width 1) (layer "B.Cu") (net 2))
 (segment (start 175.7269 40.1732) (end 175.7269 40.1731) (width 1) (layer "B.Cu") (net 2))
 (segment (start 107.442 99.314) (end 107.442 43.942) (width 1) (layer "B.Cu") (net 2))
 (segment (start 145.3782 119.38) (end 146.63 119.38) (width 1) (layer "B.Cu") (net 2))
 (segment (start 155.956 55.88) (end 157.734 54.102) (width 1) (layer "B.Cu") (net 2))
 (segment (start 107.442 43.942) (end 100.584 37.084) (width 1) (layer "B.Cu") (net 2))
 (segment (start 86.6771 40.64) (end 80.295706 40.64) (width 1) (layer "B.Cu") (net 2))
 (segment (start 148.1947 120.9447) (end 146.63 119.38) (width 1) (layer "B.Cu") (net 2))
 (segment (start 205.232 93.726) (end 205.232 88.382) (width 1) (layer "B.Cu") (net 2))
 (segment (start 86.36 30.48) (end 87.9919 32.1119) (width 1) (layer "B.Cu") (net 2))
 (segment (start 87.9919 32.1119) (end 105.3777 32.1119) (width 1) (layer "B.Cu") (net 2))
 (segment (start 80.77055 30.48) (end 86.36 30.48) (width 1) (layer "B.Cu") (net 2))
 (segment (start 146.83 51.41) (end 146.83 51.7098) (width 1) (layer "B.Cu") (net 2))
 (segment (start 80.295706 40.64) (end 78.74 39.084294) (width 1) (layer "B.Cu") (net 2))
 (segment (start 206.064 94.558) (end 205.232 93.726) (width 1) (layer "B.Cu") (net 2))
 (segment (start 221.742 81.788) (end 208.972 94.558) (width 1) (layer "B.Cu") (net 2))
 (segment (start 142.93 119.38) (end 140.898 121.412) (width 1) (layer "B.Cu") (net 2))
 (segment (start 158.4553 120.9447) (end 148.1947 120.9447) (width 1) (layer "B.Cu") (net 2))
 (segment (start 205.232 88.382) (end 194.32 77.47) (width 1) (layer "B.Cu") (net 2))
 (segment (start 221.742 48.4823) (end 221.742 81.788) (width 1) (layer "B.Cu") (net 2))
 (segment (start 129.54 121.412) (end 107.442 99.314) (width 1) (layer "B.Cu") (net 2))
 (segment (start 78.74 32.51055) (end 80.77055 30.48) (width 1) (layer "B.Cu") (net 2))
 (segment (start 208.972 94.558) (end 206.064 94.558) (width 1) (layer "B.Cu") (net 2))
 (segment (start 100.584 37.084) (end 90.2331 37.084) (width 1) (layer "B.Cu") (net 2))
 (segment (start 209.7849 36.5252) (end 221.742 48.4823) (width 1) (layer "B.Cu") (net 2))
 (segment (start 149.5 55.88) (end 155.956 55.88) (width 1) (layer "B.Cu") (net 2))
 (segment (start 146.83 51.7098) (end 146.83 53.21) (width 1) (layer "B.Cu") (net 2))
 (segment (start 98.552 76.2) (end 81.6652 59.3132) (width 1) (layer "B.Cu") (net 7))
 (segment (start 99.568 40.386) (end 97.79 38.608) (width 1) (layer "B.Cu") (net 7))
 (segment (start 101.6 76.2) (end 98.552 76.2) (width 1) (layer "B.Cu") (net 7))
 (segment (start 81.6652 58.4509) (end 85.6106 54.5055) (width 1) (layer "B.Cu") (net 7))
 (segment (start 238.506 72.898) (end 233.426 67.818) (width 1) (layer "B.Cu") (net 7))
 (segment (start 86.9725 54.5055) (end 99.568 41.91) (width 1) (layer "B.Cu") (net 7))
 (segment (start 154.94 33.8601) (end 154.94 33.02) (width 1) (layer "B.Cu") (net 7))
 (segment (start 85.6106 54.5055) (end 86.9725 54.5055) (width 1) (layer "B.Cu") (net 7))
 (segment (start 76.2 30.418) (end 78.678 27.94) (width 1) (layer "B.Cu") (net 7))
 (segment (start 76.2 40.710675) (end 76.2 30.418) (width 1) (layer "B.Cu") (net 7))
 (segment (start 198.12 103.632) (end 228.346 103.632) (width 1) (layer "B.Cu") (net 7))
 (segment (start 196.088 101.6) (end 198.12 103.632) (width 1) (layer "B.Cu") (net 7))
 (segment (start 90.678 43.18) (end 78.669325 43.18) (width 1) (layer "B.Cu") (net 7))
 (segment (start 81.3509 58.4509) (end 81.6652 58.4509) (width 1) (layer "B.Cu") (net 7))
 (segment (start 154.94 33.02) (end 152.95 33.02) (width 1) (layer "B.Cu") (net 7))
 (segment (start 154.45 51.41) (end 154.45 36.49) (width 1) (layer "B.Cu") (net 7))
 (segment (start 233.426 46.736) (end 219.71 33.02) (width 1) (layer "B.Cu") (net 7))
 (segment (start 81.6652 59.3132) (end 81.6652 58.4509) (width 1) (layer "B.Cu") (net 7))
 (segment (start 152.95 33.02) (end 152.95 32.025) (width 1) (layer "B.Cu") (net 7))
 (segment (start 94.35 27.94) (end 96.52 30.11) (width 1) (layer "B.Cu") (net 7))
 (segment (start 152.95 32.025) (end 151.035 30.11) (width 1) (layer "B.Cu") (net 7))
 (segment (start 194.32 92.71) (end 194.818 92.71) (width 1) (layer "B.Cu") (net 7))
 (segment (start 154.45 36.49) (end 154.94 36) (width 1) (layer "B.Cu") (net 7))
 (segment (start 238.506 93.472) (end 238.506 72.898) (width 1) (layer "B.Cu") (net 7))
 (segment (start 99.568 41.91) (end 99.568 40.386) (width 1) (layer "B.Cu") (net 7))
 (segment (start 154.94 33.8601) (end 154.94 36) (width 1) (layer "B.Cu") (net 7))
 (segment (start 78.669325 43.18) (end 76.2 40.710675) (width 1) (layer "B.Cu") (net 7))
 (segment (start 95.25 38.608) (end 90.678 43.18) (width 1) (layer "B.Cu") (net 7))
 (segment (start 219.71 33.02) (end 154.94 33.02) (width 1) (layer "B.Cu") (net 7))
 (segment (start 196.088 93.98) (end 196.088 101.6) (width 1) (layer "B.Cu") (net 7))
 (segment (start 233.426 67.818) (end 233.426 46.736) (width 1) (layer "B.Cu") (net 7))
 (segment (start 97.79 38.608) (end 95.25 38.608) (width 1) (layer "B.Cu") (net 7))
 (segment (start 228.346 103.632) (end 238.506 93.472) (width 1) (layer "B.Cu") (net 7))
 (segment (start 151.035 30.11) (end 96.52 30.11) (width 1) (layer "B.Cu") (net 7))
 (segment (start 81.32 58.42) (end 81.3509 58.4509) (width 1) (layer "B.Cu") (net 7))
 (segment (start 78.678 27.94) (end 94.35 27.94) (width 1) (layer "B.Cu") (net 7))
 (segment (start 194.818 92.71) (end 196.088 93.98) (width 1) (layer "B.Cu") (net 7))
 (segment (start 172.23 51.41) (end 172.23 50.528) (width 1) (layer "B.Cu") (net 19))
 (segment (start 182.88 39.95) (end 182.88 38.1) (width 1) (layer "B.Cu") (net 19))
 (segment (start 182.808 39.95) (end 182.88 39.95) (width 1) (layer "B.Cu") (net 19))
 (segment (start 172.23 50.528) (end 182.808 39.95) (width 1) (layer "B.Cu") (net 19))
 (segment (start 144.78 114.99) (end 156.99 102.78) (width 1) (layer "B.Cu") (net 35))
 (segment (start 144.78 116.84) (end 144.78 114.99) (width 1) (layer "B.Cu") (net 35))
 (segment (start 156.99 102.78) (end 156.99 99.67) (width 1) (layer "B.Cu") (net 35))
 (segment (start 216.5393 46.7081) (end 217.4419 47.6107) (width 1) (layer "B.Cu") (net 13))
 (segment (start 205.5072 75.9572) (end 207.02 77.47) (width 1) (layer "B.Cu") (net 13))
 (segment (start 205.5072 71.8568) (end 205.5072 75.9572) (width 1) (layer "B.Cu") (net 13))
 (segment (start 194.343 46.7081) (end 216.5393 46.7081) (width 1) (layer "B.Cu") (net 13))
 (segment (start 145.31 95.7411) (end 194.343 46.7081) (width 1) (layer "B.Cu") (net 13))
 (segment (start 217.4419 47.6107) (end 217.4419 59.9221) (width 1) (layer "B.Cu") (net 13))
 (segment (start 217.4419 59.9221) (end 205.5072 71.8568) (width 1) (layer "B.Cu") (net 13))
 (segment (start 145.31 99.67) (end 145.31 95.7411) (width 1) (layer "B.Cu") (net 13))
 (segment (start 207.02 73.13) (end 218.6447 61.5053) (width 1) (layer "B.Cu") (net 14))
 (segment (start 218.6447 47.0847) (end 217.049 45.489) (width 1) (layer "B.Cu") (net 14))
 (segment (start 207.02 74.93) (end 207.02 73.13) (width 1) (layer "B.Cu") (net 14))
 (segment (start 142.77 94.212) (end 142.77 99.67) (width 1) (layer "B.Cu") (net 14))
 (segment (start 191.493 45.489) (end 142.77 94.212) (width 1) (layer "B.Cu") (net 14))
 (segment (start 218.6447 61.5053) (end 218.6447 47.0847) (width 1) (layer "B.Cu") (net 14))
 (segment (start 217.049 45.489) (end 191.493 45.489) (width 1) (layer "B.Cu") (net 14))
 (segment (start 147.85 95.99) (end 195.58 48.26) (width 1) (layer "B.Cu") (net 18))
 (segment (start 147.85 99.67) (end 147.85 95.99) (width 1) (layer "B.Cu") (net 18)))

